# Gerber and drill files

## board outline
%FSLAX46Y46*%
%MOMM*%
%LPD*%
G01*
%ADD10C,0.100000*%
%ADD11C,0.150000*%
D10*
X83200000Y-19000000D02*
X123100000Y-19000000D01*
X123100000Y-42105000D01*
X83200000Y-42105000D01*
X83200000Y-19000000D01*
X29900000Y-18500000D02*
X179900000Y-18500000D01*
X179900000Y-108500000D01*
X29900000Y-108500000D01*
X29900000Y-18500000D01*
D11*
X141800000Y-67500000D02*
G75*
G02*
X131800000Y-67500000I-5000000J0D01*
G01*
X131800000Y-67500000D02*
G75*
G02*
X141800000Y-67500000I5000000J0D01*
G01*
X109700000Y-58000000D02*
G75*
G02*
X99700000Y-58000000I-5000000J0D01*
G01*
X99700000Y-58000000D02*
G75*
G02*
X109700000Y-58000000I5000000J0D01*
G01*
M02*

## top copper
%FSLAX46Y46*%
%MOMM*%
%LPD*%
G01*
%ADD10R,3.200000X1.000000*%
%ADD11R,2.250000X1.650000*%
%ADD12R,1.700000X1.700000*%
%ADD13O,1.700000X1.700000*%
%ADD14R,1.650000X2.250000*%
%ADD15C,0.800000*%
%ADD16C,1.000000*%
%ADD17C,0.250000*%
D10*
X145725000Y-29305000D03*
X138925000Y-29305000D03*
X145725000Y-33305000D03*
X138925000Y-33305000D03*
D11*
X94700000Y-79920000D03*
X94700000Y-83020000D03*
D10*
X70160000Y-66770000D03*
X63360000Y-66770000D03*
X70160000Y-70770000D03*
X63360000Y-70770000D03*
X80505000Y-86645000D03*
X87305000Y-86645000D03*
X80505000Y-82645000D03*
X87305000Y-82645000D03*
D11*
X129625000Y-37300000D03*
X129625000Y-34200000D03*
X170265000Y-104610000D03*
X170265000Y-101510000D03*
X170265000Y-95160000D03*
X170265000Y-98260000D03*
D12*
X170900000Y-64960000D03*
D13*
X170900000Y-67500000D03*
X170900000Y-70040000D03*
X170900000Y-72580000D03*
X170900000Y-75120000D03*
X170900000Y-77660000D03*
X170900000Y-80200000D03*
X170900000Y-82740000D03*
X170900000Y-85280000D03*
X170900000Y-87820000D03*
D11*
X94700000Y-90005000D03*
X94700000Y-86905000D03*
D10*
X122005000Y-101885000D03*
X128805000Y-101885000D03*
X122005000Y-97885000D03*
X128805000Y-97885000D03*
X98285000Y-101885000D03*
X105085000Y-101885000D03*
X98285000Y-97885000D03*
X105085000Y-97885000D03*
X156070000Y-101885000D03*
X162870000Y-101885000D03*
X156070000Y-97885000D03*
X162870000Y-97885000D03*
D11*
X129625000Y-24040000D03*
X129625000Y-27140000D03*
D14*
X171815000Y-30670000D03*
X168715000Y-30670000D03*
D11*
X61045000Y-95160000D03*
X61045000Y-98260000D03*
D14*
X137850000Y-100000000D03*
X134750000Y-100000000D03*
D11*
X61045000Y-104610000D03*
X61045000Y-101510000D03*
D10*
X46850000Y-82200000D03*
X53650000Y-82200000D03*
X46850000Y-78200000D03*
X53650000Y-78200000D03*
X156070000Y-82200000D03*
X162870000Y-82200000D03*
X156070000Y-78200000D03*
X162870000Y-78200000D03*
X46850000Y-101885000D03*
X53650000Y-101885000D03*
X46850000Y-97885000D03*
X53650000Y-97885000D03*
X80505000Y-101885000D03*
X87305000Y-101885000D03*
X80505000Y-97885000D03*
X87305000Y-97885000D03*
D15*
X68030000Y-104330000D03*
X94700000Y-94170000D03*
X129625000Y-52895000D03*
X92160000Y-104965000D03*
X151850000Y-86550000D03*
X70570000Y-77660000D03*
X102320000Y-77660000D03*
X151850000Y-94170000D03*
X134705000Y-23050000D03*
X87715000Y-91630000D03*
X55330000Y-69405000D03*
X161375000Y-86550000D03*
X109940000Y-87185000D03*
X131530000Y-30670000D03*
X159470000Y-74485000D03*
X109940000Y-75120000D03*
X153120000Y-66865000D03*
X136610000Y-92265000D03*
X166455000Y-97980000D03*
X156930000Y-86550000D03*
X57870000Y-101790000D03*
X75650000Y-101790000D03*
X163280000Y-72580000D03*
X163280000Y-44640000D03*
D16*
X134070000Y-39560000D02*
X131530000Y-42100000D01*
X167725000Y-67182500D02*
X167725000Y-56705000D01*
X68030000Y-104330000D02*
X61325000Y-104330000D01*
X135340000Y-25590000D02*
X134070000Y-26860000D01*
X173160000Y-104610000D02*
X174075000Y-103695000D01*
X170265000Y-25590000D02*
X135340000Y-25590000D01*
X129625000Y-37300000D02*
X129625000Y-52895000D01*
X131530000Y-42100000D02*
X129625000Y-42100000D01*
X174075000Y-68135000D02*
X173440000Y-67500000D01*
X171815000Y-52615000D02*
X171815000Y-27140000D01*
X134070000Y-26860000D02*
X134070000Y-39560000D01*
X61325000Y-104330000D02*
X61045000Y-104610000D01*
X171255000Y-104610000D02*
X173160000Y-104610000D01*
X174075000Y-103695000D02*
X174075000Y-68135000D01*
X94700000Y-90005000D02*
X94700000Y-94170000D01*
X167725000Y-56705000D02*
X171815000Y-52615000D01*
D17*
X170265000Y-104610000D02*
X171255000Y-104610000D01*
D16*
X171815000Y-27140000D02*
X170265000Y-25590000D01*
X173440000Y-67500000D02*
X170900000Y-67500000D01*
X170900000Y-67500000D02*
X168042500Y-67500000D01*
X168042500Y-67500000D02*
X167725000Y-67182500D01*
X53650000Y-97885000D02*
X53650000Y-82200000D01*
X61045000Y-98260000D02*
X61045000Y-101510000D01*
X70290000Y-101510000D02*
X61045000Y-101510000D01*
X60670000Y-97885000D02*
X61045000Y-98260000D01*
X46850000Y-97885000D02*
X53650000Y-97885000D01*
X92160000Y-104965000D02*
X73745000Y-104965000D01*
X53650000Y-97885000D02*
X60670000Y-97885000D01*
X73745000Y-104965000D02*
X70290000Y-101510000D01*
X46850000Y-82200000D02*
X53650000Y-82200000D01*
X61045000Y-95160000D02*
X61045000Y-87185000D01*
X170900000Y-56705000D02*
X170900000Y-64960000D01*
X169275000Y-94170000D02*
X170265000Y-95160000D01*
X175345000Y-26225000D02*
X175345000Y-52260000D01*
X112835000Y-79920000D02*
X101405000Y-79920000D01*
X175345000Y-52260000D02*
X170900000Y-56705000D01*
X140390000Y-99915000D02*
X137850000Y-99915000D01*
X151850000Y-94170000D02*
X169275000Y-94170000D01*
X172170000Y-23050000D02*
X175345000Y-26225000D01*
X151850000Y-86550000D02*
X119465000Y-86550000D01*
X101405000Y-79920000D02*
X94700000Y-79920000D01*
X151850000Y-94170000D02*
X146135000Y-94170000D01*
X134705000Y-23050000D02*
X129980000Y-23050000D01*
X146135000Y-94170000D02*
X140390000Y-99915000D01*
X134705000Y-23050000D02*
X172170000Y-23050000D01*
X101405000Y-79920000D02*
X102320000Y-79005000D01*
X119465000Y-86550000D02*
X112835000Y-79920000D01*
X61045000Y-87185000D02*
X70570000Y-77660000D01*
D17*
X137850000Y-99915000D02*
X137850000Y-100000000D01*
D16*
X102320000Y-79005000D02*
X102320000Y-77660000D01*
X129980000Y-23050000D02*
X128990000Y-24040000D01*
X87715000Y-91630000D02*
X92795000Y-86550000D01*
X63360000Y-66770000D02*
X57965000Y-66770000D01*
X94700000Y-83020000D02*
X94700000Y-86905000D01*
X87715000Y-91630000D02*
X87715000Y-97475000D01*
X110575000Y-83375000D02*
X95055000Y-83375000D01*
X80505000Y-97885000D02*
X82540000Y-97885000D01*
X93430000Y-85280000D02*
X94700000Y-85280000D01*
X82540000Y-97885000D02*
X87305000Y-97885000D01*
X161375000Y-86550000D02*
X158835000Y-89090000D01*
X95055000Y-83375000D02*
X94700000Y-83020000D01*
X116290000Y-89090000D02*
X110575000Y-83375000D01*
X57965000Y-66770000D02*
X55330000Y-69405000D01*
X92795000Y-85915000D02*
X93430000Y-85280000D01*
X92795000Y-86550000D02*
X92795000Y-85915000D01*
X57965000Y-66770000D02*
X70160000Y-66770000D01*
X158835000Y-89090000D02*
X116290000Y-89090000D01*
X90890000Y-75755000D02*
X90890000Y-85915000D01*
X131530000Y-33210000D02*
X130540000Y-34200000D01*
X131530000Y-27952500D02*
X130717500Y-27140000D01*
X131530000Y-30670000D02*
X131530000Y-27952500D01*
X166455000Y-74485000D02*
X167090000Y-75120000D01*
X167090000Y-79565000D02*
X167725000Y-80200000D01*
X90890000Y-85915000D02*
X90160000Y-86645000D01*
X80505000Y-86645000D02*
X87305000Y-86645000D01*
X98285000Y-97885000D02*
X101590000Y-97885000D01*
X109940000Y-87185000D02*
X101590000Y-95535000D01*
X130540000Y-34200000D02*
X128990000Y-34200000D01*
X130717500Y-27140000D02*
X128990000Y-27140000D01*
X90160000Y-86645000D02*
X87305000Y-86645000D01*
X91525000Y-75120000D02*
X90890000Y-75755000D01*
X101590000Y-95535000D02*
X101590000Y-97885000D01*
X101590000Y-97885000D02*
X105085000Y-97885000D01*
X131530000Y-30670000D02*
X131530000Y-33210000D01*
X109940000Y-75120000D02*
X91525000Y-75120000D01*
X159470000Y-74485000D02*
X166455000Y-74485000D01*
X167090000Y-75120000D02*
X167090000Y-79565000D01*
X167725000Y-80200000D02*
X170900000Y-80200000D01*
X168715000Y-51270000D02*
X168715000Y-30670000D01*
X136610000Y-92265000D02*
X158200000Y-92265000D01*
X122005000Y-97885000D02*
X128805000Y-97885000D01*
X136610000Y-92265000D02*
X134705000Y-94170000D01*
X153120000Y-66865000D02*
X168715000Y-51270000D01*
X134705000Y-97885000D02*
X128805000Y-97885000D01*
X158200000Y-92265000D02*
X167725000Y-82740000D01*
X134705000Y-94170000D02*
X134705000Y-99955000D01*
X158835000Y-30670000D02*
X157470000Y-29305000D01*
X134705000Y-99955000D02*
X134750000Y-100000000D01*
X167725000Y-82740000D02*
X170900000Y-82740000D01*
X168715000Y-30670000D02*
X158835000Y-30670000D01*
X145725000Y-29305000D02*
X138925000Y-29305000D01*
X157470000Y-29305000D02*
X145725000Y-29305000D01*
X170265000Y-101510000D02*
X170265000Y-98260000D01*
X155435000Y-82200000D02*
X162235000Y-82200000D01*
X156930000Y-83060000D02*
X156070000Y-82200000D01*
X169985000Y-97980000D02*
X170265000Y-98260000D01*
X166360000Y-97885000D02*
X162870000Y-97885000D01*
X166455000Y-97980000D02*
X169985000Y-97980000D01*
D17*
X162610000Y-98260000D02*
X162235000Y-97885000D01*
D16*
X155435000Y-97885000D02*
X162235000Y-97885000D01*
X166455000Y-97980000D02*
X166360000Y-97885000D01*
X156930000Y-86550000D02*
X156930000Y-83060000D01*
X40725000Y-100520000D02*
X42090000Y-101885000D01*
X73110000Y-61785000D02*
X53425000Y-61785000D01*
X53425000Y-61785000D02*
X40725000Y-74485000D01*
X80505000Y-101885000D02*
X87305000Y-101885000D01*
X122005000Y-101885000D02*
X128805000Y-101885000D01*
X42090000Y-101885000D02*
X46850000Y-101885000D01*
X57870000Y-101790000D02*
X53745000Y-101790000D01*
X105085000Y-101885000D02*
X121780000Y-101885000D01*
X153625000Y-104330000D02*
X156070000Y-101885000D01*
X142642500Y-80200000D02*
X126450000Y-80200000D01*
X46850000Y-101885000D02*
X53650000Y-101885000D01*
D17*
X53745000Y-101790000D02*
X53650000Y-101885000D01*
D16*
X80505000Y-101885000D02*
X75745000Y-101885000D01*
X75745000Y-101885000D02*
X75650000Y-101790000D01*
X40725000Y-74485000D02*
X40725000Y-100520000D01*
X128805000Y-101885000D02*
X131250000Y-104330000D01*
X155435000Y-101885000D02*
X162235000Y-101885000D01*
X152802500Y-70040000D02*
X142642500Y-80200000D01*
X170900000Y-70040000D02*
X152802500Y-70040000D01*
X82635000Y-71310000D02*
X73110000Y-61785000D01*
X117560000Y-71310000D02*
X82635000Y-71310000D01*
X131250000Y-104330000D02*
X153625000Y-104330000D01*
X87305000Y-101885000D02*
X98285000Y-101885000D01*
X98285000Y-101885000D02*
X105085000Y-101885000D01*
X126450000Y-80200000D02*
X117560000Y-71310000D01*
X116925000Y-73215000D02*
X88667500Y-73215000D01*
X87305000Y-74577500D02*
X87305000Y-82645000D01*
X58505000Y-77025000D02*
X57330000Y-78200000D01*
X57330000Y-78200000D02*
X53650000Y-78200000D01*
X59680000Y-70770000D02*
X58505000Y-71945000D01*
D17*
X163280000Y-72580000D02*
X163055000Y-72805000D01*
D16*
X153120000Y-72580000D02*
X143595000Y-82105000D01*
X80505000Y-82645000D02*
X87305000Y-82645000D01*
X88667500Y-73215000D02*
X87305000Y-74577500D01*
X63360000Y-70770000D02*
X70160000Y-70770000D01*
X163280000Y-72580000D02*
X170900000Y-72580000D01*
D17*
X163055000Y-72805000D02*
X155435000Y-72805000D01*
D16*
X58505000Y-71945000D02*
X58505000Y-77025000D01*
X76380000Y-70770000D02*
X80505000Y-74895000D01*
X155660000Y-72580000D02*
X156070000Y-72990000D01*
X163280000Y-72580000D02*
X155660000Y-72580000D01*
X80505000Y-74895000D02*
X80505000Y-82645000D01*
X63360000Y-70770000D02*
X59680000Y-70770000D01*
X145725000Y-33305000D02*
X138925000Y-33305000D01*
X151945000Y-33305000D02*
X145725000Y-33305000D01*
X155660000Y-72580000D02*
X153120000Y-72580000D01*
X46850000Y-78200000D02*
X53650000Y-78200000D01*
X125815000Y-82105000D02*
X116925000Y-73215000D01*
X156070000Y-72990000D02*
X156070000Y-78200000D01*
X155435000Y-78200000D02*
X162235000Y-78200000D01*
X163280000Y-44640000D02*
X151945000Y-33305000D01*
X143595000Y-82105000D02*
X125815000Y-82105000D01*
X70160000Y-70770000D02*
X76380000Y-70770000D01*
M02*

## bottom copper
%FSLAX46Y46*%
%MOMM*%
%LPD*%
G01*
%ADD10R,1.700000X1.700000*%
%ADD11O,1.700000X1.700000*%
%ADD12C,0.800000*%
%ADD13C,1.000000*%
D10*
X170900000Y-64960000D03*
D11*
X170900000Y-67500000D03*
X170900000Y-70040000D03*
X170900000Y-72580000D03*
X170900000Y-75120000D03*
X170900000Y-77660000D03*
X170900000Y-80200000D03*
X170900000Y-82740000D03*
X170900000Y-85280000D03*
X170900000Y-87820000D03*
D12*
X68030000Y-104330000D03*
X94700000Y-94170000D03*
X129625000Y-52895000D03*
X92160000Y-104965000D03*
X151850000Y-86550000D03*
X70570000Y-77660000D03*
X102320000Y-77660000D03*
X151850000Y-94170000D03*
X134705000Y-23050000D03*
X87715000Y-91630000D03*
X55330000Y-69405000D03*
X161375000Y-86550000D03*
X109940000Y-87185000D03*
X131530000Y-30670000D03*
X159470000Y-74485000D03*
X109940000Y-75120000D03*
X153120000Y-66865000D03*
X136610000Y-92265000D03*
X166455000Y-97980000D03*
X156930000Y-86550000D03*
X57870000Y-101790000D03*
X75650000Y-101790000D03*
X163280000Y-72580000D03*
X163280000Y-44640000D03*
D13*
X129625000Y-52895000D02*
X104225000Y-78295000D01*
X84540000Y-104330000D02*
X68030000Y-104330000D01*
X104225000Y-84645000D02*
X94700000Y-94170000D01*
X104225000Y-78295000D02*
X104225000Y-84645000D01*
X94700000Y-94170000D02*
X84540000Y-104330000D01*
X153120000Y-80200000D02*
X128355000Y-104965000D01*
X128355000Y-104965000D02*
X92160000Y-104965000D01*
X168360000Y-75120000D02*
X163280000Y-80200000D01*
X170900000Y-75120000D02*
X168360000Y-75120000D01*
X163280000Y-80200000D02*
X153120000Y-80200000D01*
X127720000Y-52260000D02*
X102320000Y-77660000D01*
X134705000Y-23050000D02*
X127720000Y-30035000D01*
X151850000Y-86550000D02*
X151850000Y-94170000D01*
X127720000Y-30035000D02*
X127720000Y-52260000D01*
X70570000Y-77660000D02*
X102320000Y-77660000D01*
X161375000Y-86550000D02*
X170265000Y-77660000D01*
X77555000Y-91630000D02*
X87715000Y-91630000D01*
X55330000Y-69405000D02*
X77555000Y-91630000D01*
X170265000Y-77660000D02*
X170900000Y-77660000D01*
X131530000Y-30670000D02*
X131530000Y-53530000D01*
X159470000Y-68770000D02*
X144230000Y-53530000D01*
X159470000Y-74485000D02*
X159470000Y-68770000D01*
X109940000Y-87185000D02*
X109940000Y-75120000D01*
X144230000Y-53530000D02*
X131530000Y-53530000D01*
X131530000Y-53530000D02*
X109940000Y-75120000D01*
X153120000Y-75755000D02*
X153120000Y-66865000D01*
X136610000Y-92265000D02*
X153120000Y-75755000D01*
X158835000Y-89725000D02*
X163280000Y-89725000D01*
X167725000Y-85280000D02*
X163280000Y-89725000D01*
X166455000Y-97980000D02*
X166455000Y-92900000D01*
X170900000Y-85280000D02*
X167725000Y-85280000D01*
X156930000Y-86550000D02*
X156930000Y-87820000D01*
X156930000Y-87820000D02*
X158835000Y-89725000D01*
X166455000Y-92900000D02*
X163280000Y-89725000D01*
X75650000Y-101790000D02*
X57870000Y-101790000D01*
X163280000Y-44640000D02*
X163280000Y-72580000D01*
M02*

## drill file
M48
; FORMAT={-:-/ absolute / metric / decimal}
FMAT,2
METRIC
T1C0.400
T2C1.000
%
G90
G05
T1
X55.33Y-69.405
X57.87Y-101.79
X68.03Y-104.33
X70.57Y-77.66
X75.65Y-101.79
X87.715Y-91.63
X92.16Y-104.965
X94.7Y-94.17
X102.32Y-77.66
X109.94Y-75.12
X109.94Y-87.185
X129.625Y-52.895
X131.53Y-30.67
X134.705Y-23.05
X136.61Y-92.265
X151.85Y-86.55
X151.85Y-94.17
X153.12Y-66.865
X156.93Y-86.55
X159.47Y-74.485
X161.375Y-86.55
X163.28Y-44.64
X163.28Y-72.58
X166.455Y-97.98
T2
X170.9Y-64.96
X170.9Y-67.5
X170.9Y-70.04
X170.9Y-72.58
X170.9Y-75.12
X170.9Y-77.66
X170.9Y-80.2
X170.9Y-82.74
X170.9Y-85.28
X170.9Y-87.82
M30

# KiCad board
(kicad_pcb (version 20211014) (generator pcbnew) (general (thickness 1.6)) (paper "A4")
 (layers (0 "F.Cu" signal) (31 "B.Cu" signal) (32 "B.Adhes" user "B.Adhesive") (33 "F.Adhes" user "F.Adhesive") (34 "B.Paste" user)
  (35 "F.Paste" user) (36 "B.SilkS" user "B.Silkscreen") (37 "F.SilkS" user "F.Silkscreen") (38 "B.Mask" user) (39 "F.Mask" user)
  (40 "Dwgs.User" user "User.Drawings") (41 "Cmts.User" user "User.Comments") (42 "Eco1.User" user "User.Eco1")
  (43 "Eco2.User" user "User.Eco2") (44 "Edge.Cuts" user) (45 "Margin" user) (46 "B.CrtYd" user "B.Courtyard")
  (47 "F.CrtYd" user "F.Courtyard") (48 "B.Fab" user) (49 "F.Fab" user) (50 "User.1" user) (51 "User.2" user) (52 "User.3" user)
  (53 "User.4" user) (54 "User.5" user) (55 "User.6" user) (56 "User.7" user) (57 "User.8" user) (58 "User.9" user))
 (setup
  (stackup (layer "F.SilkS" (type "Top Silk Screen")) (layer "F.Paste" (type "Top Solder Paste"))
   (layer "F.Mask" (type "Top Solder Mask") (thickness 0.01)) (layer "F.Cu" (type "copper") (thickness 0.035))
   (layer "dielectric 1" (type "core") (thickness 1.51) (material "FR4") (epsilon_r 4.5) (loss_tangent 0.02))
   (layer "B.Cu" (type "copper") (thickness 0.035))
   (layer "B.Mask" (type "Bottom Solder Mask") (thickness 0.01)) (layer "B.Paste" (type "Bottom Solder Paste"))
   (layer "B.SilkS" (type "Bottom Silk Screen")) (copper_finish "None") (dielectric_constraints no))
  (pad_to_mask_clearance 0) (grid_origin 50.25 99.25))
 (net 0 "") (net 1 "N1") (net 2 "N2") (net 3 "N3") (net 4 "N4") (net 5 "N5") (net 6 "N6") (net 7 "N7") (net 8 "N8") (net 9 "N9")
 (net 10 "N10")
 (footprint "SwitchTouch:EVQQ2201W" (layer "F.Cu") (at 142.325 31.305 180)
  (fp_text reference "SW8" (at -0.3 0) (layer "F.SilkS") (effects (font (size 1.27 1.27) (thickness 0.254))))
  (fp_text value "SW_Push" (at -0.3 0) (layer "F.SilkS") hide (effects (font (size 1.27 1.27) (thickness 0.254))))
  (pad "A1" smd rect locked (at -3.4 2 270) (size 1 3.2) (layers "F.Cu" "F.Paste" "F.Mask") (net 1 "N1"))
  (pad "A2" smd rect locked (at 3.4 2 270) (size 1 3.2) (layers "F.Cu" "F.Paste" "F.Mask") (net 1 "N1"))
  (pad "B1" smd rect locked (at -3.4 -2 270) (size 1 3.2) (layers "F.Cu" "F.Paste" "F.Mask") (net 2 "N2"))
  (pad "B2" smd rect locked (at 3.4 -2 270) (size 1 3.2) (layers "F.Cu" "F.Paste" "F.Mask") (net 2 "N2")))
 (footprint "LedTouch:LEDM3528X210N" (layer "F.Cu") (at 94.7 81.47 -90)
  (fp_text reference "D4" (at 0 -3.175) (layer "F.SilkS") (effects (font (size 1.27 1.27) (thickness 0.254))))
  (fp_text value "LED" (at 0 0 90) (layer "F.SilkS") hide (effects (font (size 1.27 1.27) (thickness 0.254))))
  (pad "1" smd rect locked (at -1.55 0 270) (size 1.65 2.25) (layers "F.Cu" "F.Paste" "F.Mask") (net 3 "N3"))
  (pad "2" smd rect locked (at 1.55 0 270) (size 1.65 2.25) (layers "F.Cu" "F.Paste" "F.Mask") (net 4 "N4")))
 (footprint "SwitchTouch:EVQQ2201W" (layer "F.Cu") (at 66.76 68.77 180)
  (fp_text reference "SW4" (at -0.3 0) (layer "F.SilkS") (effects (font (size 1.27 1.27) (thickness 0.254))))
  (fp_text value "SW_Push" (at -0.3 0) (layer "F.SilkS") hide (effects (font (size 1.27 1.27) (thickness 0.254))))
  (pad "A1" smd rect locked (at -3.4 2 270) (size 1 3.2) (layers "F.Cu" "F.Paste" "F.Mask") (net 4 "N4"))
  (pad "A2" smd rect locked (at 3.4 2 270) (size 1 3.2) (layers "F.Cu" "F.Paste" "F.Mask") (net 4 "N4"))
  (pad "B1" smd rect locked (at -3.4 -2 270) (size 1 3.2) (layers "F.Cu" "F.Paste" "F.Mask") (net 2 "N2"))
  (pad "B2" smd rect locked (at 3.4 -2 270) (size 1 3.2) (layers "F.Cu" "F.Paste" "F.Mask") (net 2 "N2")))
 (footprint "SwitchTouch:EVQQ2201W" (layer "F.Cu") (at 83.905 84.645)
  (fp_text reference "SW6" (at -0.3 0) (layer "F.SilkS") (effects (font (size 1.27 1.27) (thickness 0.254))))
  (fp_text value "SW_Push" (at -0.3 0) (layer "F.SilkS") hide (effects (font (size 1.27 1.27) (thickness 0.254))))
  (pad "A1" smd rect locked (at -3.4 2 90) (size 1 3.2) (layers "F.Cu" "F.Paste" "F.Mask") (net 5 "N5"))
  (pad "A2" smd rect locked (at 3.4 2 90) (size 1 3.2) (layers "F.Cu" "F.Paste" "F.Mask") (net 5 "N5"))
  (pad "B1" smd rect locked (at -3.4 -2 90) (size 1 3.2) (layers "F.Cu" "F.Paste" "F.Mask") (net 2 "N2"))
  (pad "B2" smd rect locked (at 3.4 -2 90) (size 1 3.2) (layers "F.Cu" "F.Paste" "F.Mask") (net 2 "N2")))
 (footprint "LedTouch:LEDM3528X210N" (layer "F.Cu") (at 129.625 35.75 90)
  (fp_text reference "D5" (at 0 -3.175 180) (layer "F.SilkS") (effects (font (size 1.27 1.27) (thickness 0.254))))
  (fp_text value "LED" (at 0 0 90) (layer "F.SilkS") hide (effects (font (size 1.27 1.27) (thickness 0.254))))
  (pad "1" smd rect locked (at -1.55 0 90) (size 1.65 2.25) (layers "F.Cu" "F.Paste" "F.Mask") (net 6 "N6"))
  (pad "2" smd rect locked (at 1.55 0 90) (size 1.65 2.25) (layers "F.Cu" "F.Paste" "F.Mask") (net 5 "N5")))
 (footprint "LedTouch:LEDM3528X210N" (layer "F.Cu") (at 170.265 103.06 90)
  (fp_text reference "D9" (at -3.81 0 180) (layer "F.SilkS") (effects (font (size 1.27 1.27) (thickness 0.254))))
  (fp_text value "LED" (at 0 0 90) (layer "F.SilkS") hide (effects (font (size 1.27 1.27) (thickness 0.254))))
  (pad "1" smd rect locked (at -1.55 0 90) (size 1.65 2.25) (layers "F.Cu" "F.Paste" "F.Mask") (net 6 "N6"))
  (pad "2" smd rect locked (at 1.55 0 90) (size 1.65 2.25) (layers "F.Cu" "F.Paste" "F.Mask") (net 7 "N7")))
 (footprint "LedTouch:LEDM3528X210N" (layer "F.Cu") (at 170.265 96.71 -90)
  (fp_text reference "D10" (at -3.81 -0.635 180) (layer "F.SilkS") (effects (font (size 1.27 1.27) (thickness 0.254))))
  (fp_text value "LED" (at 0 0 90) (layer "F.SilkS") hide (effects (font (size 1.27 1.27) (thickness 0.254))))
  (pad "1" smd rect locked (at -1.55 0 270) (size 1.65 2.25) (layers "F.Cu" "F.Paste" "F.Mask") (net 3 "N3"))
  (pad "2" smd rect locked (at 1.55 0 270) (size 1.65 2.25) (layers "F.Cu" "F.Paste" "F.Mask") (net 7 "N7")))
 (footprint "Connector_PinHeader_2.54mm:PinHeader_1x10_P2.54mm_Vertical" (layer "F.Cu") (at 170.9 64.96)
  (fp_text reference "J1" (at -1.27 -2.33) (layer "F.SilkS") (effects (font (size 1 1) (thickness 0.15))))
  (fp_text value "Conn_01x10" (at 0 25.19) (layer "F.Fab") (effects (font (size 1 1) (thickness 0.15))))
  (pad "1" thru_hole rect (at 0 0) (size 1.7 1.7) (drill 1) (layers *.Cu *.Mask) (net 3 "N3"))
  (pad "2" thru_hole oval (at 0 2.54) (size 1.7 1.7) (drill 1) (layers *.Cu *.Mask) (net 6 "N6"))
  (pad "3" thru_hole oval (at 0 5.08) (size 1.7 1.7) (drill 1) (layers *.Cu *.Mask) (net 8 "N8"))
  (pad "4" thru_hole oval (at 0 7.62) (size 1.7 1.7) (drill 1) (layers *.Cu *.Mask) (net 2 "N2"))
  (pad "5" thru_hole oval (at 0 10.16) (size 1.7 1.7) (drill 1) (layers *.Cu *.Mask) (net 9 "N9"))
  (pad "6" thru_hole oval (at 0 12.7) (size 1.7 1.7) (drill 1) (layers *.Cu *.Mask) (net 4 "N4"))
  (pad "7" thru_hole oval (at 0 15.24) (size 1.7 1.7) (drill 1) (layers *.Cu *.Mask) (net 5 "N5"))
  (pad "8" thru_hole oval (at 0 17.78) (size 1.7 1.7) (drill 1) (layers *.Cu *.Mask) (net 1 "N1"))
  (pad "9" thru_hole oval (at 0 20.32) (size 1.7 1.7) (drill 1) (layers *.Cu *.Mask) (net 7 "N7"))
  (pad "10" thru_hole oval (at 0 22.86) (size 1.7 1.7) (drill 1) (layers *.Cu *.Mask) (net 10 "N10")))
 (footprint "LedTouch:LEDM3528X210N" (layer "F.Cu") (at 94.7 88.455 90)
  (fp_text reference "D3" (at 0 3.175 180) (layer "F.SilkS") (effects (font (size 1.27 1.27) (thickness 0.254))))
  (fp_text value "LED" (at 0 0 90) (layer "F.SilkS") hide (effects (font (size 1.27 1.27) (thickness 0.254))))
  (pad "1" smd rect locked (at -1.55 0 90) (size 1.65 2.25) (layers "F.Cu" "F.Paste" "F.Mask") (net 6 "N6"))
  (pad "2" smd rect locked (at 1.55 0 90) (size 1.65 2.25) (layers "F.Cu" "F.Paste" "F.Mask") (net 4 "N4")))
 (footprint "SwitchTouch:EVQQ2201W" (layer "F.Cu") (at 125.405 99.885)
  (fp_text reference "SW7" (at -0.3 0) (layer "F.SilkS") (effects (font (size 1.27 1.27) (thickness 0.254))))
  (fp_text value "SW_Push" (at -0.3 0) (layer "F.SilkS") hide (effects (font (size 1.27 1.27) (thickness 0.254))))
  (pad "A1" smd rect locked (at -3.4 2 90) (size 1 3.2) (layers "F.Cu" "F.Paste" "F.Mask") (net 8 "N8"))
  (pad "A2" smd rect locked (at 3.4 2 90) (size 1 3.2) (layers "F.Cu" "F.Paste" "F.Mask") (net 8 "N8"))
  (pad "B1" smd rect locked (at -3.4 -2 90) (size 1 3.2) (layers "F.Cu" "F.Paste" "F.Mask") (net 1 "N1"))
  (pad "B2" smd rect locked (at 3.4 -2 90) (size 1 3.2) (layers "F.Cu" "F.Paste" "F.Mask") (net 1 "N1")))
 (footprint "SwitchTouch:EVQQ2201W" (layer "F.Cu") (at 101.685 99.885)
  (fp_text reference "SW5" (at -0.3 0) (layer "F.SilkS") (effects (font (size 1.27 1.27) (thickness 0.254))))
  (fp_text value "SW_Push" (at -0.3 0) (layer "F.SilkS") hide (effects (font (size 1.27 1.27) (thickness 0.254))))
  (pad "A1" smd rect locked (at -3.4 2 90) (size 1 3.2) (layers "F.Cu" "F.Paste" "F.Mask") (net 8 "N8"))
  (pad "A2" smd rect locked (at 3.4 2 90) (size 1 3.2) (layers "F.Cu" "F.Paste" "F.Mask") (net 8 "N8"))
  (pad "B1" smd rect locked (at -3.4 -2 90) (size 1 3.2) (layers "F.Cu" "F.Paste" "F.Mask") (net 5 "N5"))
  (pad "B2" smd rect locked (at 3.4 -2 90) (size 1 3.2) (layers "F.Cu" "F.Paste" "F.Mask") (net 5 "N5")))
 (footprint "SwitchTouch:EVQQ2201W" (layer "F.Cu") (at 159.47 99.885)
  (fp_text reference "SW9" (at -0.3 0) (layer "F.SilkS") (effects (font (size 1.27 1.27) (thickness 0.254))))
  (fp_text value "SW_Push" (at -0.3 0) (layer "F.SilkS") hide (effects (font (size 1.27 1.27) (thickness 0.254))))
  (pad "A1" smd rect locked (at -3.4 2 90) (size 1 3.2) (layers "F.Cu" "F.Paste" "F.Mask") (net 8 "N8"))
  (pad "A2" smd rect locked (at 3.4 2 90) (size 1 3.2) (layers "F.Cu" "F.Paste" "F.Mask") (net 8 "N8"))
  (pad "B1" smd rect locked (at -3.4 -2 90) (size 1 3.2) (layers "F.Cu" "F.Paste" "F.Mask") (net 7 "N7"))
  (pad "B2" smd rect locked (at 3.4 -2 90) (size 1 3.2) (layers "F.Cu" "F.Paste" "F.Mask") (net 7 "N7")))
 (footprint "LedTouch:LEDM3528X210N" (layer "F.Cu") (at 129.625 25.59 -90)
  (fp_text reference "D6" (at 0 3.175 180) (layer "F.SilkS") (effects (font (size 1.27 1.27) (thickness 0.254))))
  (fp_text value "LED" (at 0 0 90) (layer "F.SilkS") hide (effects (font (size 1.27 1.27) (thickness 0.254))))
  (pad "1" smd rect locked (at -1.55 0 270) (size 1.65 2.25) (layers "F.Cu" "F.Paste" "F.Mask") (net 3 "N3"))
  (pad "2" smd rect locked (at 1.55 0 270) (size 1.65 2.25) (layers "F.Cu" "F.Paste" "F.Mask") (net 5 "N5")))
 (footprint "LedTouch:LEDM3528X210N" (layer "F.Cu") (at 170.265 30.67 180)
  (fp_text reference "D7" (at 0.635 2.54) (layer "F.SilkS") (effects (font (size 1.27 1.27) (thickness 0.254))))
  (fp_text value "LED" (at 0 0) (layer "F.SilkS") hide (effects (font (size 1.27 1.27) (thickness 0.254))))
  (pad "1" smd rect locked (at -1.55 0 180) (size 1.65 2.25) (layers "F.Cu" "F.Paste" "F.Mask") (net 6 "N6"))
  (pad "2" smd rect locked (at 1.55 0 180) (size 1.65 2.25) (layers "F.Cu" "F.Paste" "F.Mask") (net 1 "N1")))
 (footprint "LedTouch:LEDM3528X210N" (layer "F.Cu") (at 61.045 96.71 -90)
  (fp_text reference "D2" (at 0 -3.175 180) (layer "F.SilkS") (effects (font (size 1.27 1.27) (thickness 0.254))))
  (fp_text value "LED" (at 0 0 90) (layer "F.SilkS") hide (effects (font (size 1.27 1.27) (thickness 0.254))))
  (pad "1" smd rect locked (at -1.55 0 270) (size 1.65 2.25) (layers "F.Cu" "F.Paste" "F.Mask") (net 3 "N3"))
  (pad "2" smd rect locked (at 1.55 0 270) (size 1.65 2.25) (layers "F.Cu" "F.Paste" "F.Mask") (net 9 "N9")))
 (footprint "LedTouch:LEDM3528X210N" (layer "F.Cu") (at 136.3 100 180)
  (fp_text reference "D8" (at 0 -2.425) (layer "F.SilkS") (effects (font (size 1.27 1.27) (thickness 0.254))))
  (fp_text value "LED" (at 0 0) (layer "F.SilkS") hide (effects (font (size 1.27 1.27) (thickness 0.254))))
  (pad "1" smd rect locked (at -1.55 0 180) (size 1.65 2.25) (layers "F.Cu" "F.Paste" "F.Mask") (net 3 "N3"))
  (pad "2" smd rect locked (at 1.55 0 180) (size 1.65 2.25) (layers "F.Cu" "F.Paste" "F.Mask") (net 1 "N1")))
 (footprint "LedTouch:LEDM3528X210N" (layer "F.Cu") (at 61.045 103.06 90)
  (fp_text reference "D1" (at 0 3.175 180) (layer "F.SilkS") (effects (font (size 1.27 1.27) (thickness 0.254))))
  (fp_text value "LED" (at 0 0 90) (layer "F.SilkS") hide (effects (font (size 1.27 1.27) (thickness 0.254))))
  (pad "1" smd rect locked (at -1.55 0 90) (size 1.65 2.25) (layers "F.Cu" "F.Paste" "F.Mask") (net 6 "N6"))
  (pad "2" smd rect locked (at 1.55 0 90) (size 1.65 2.25) (layers "F.Cu" "F.Paste" "F.Mask") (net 9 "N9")))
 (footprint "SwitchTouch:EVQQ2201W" (layer "F.Cu") (at 50.25 80.2)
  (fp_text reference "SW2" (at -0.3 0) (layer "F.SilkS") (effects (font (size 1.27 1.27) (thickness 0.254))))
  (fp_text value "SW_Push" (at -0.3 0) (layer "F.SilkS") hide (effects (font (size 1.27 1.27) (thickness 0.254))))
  (pad "A1" smd rect locked (at -3.4 2 90) (size 1 3.2) (layers "F.Cu" "F.Paste" "F.Mask") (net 9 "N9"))
  (pad "A2" smd rect locked (at 3.4 2 90) (size 1 3.2) (layers "F.Cu" "F.Paste" "F.Mask") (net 9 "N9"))
  (pad "B1" smd rect locked (at -3.4 -2 90) (size 1 3.2) (layers "F.Cu" "F.Paste" "F.Mask") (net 2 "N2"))
  (pad "B2" smd rect locked (at 3.4 -2 90) (size 1 3.2) (layers "F.Cu" "F.Paste" "F.Mask") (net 2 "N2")))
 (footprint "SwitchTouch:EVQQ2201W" (layer "F.Cu") (at 159.47 80.2)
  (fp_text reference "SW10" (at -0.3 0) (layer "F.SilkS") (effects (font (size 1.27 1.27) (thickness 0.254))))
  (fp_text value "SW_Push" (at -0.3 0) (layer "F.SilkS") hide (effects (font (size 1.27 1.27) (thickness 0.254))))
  (pad "A1" smd rect locked (at -3.4 2 90) (size 1 3.2) (layers "F.Cu" "F.Paste" "F.Mask") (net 7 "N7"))
  (pad "A2" smd rect locked (at 3.4 2 90) (size 1 3.2) (layers "F.Cu" "F.Paste" "F.Mask") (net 7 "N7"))
  (pad "B1" smd rect locked (at -3.4 -2 90) (size 1 3.2) (layers "F.Cu" "F.Paste" "F.Mask") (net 2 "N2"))
  (pad "B2" smd rect locked (at 3.4 -2 90) (size 1 3.2) (layers "F.Cu" "F.Paste" "F.Mask") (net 2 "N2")))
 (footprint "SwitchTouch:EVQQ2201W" (layer "F.Cu") (at 50.25 99.885)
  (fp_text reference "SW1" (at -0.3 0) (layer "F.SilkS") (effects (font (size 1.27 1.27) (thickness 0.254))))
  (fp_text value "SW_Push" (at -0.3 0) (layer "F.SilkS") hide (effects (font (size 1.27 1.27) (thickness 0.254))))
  (pad "A1" smd rect locked (at -3.4 2 90) (size 1 3.2) (layers "F.Cu" "F.Paste" "F.Mask") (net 8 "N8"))
  (pad "A2" smd rect locked (at 3.4 2 90) (size 1 3.2) (layers "F.Cu" "F.Paste" "F.Mask") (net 8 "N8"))
  (pad "B1" smd rect locked (at -3.4 -2 90) (size 1 3.2) (layers "F.Cu" "F.Paste" "F.Mask") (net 9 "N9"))
  (pad "B2" smd rect locked (at 3.4 -2 90) (size 1 3.2) (layers "F.Cu" "F.Paste" "F.Mask") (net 9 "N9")))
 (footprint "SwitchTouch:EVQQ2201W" (layer "F.Cu") (at 83.905 99.885)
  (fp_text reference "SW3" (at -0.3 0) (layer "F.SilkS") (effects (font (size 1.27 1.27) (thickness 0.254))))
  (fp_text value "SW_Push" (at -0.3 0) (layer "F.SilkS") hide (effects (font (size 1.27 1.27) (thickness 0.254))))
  (pad "A1" smd rect locked (at -3.4 2 90) (size 1 3.2) (layers "F.Cu" "F.Paste" "F.Mask") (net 8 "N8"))
  (pad "A2" smd rect locked (at 3.4 2 90) (size 1 3.2) (layers "F.Cu" "F.Paste" "F.Mask") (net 8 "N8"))
  (pad "B1" smd rect locked (at -3.4 -2 90) (size 1 3.2) (layers "F.Cu" "F.Paste" "F.Mask") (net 4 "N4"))
  (pad "B2" smd rect locked (at 3.4 -2 90) (size 1 3.2) (layers "F.Cu" "F.Paste" "F.Mask") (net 4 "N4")))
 (gr_rect (start 83.2 19) (end 123.1 42.105) (layer "Edge.Cuts") (width 0.1) (fill none))
 (gr_rect (start 29.9 18.5) (end 179.9 108.5) (layer "Edge.Cuts") (width 0.1) (fill none))
 (gr_circle (center 136.8 67.5) (end 141.8 67.5) (layer "Edge.Cuts") (width 0.15) (fill none))
 (gr_circle (center 104.7 58) (end 109.7 58) (layer "Edge.Cuts") (width 0.15) (fill none))
 (segment (start 134.07 39.56) (end 131.53 42.1) (width 1) (layer "F.Cu") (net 6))
 (segment (start 167.725 67.1825) (end 167.725 56.705) (width 1) (layer "F.Cu") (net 6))
 (segment (start 68.03 104.33) (end 61.325 104.33) (width 1) (layer "F.Cu") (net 6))
 (segment (start 135.34 25.59) (end 134.07 26.86) (width 1) (layer "F.Cu") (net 6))
 (segment (start 173.16 104.61) (end 174.075 103.695) (width 1) (layer "F.Cu") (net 6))
 (segment (start 170.265 25.59) (end 135.34 25.59) (width 1) (layer "F.Cu") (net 6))
 (segment (start 129.625 37.3) (end 129.625 52.895) (width 1) (layer "F.Cu") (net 6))
 (segment (start 131.53 42.1) (end 129.625 42.1) (width 1) (layer "F.Cu") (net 6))
 (segment (start 174.075 68.135) (end 173.44 67.5) (width 1) (layer "F.Cu") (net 6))
 (segment (start 171.815 52.615) (end 171.815 27.14) (width 1) (layer "F.Cu") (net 6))
 (segment (start 134.07 26.86) (end 134.07 39.56) (width 1) (layer "F.Cu") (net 6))
 (segment (start 61.325 104.33) (end 61.045 104.61) (width 1) (layer "F.Cu") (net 6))
 (segment (start 171.255 104.61) (end 173.16 104.61) (width 1) (layer "F.Cu") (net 6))
 (segment (start 174.075 103.695) (end 174.075 68.135) (width 1) (layer "F.Cu") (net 6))
 (segment (start 94.7 90.005) (end 94.7 94.17) (width 1) (layer "F.Cu") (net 6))
 (segment (start 167.725 56.705) (end 171.815 52.615) (width 1) (layer "F.Cu") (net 6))
 (segment (start 170.265 104.61) (end 171.255 104.61) (width 0.25) (layer "F.Cu") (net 6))
 (segment (start 171.815 27.14) (end 170.265 25.59) (width 1) (layer "F.Cu") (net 6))
 (segment (start 173.44 67.5) (end 170.9 67.5) (width 1) (layer "F.Cu") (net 6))
 (segment (start 170.9 67.5) (end 168.0425 67.5) (width 1) (layer "F.Cu") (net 6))
 (segment (start 168.0425 67.5) (end 167.725 67.1825) (width 1) (layer "F.Cu") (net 6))
 (via (at 68.03 104.33) (size 0.8) (drill 0.4) (layers "F.Cu" "B.Cu") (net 6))
 (via (at 94.7 94.17) (size 0.8) (drill 0.4) (layers "F.Cu" "B.Cu") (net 6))
 (via (at 129.625 52.895) (size 0.8) (drill 0.4) (layers "F.Cu" "B.Cu") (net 6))
 (segment (start 129.625 52.895) (end 104.225 78.295) (width 1) (layer "B.Cu") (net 6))
 (segment (start 84.54 104.33) (end 68.03 104.33) (width 1) (layer "B.Cu") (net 6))
 (segment (start 104.225 84.645) (end 94.7 94.17) (width 1) (layer "B.Cu") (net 6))
 (segment (start 104.225 78.295) (end 104.225 84.645) (width 1) (layer "B.Cu") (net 6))
 (segment (start 94.7 94.17) (end 84.54 104.33) (width 1) (layer "B.Cu") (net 6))
 (segment (start 53.65 97.885) (end 53.65 82.2) (width 1) (layer "F.Cu") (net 9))
 (segment (start 61.045 98.26) (end 61.045 101.51) (width 1) (layer "F.Cu") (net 9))
 (segment (start 70.29 101.51) (end 61.045 101.51) (width 1) (layer "F.Cu") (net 9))
 (segment (start 60.67 97.885) (end 61.045 98.26) (width 1) (layer "F.Cu") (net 9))
 (segment (start 46.85 97.885) (end 53.65 97.885) (width 1) (layer "F.Cu") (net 9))
 (segment (start 92.16 104.965) (end 73.745 104.965) (width 1) (layer "F.Cu") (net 9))
 (segment (start 53.65 97.885) (end 60.67 97.885) (width 1) (layer "F.Cu") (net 9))
 (segment (start 73.745 104.965) (end 70.29 101.51) (width 1) (layer "F.Cu") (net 9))
 (segment (start 46.85 82.2) (end 53.65 82.2) (width 1) (layer "F.Cu") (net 9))
 (via (at 92.16 104.965) (size 0.8) (drill 0.4) (layers "F.Cu" "B.Cu") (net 9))
 (segment (start 153.12 80.2) (end 128.355 104.965) (width 1) (layer "B.Cu") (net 9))
 (segment (start 128.355 104.965) (end 92.16 104.965) (width 1) (layer "B.Cu") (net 9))
 (segment (start 168.36 75.12) (end 163.28 80.2) (width 1) (layer "B.Cu") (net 9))
 (segment (start 170.9 75.12) (end 168.36 75.12) (width 1) (layer "B.Cu") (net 9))
 (segment (start 163.28 80.2) (end 153.12 80.2) (width 1) (layer "B.Cu") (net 9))
 (segment (start 61.045 95.16) (end 61.045 87.185) (width 1) (layer "F.Cu") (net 3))
 (segment (start 170.9 56.705) (end 170.9 64.96) (width 1) (layer "F.Cu") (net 3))
 (segment (start 169.275 94.17) (end 170.265 95.16) (width 1) (layer "F.Cu") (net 3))
 (segment (start 175.345 26.225) (end 175.345 52.26) (width 1) (layer "F.Cu") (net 3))
 (segment (start 112.835 79.92) (end 101.405 79.92) (width 1) (layer "F.Cu") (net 3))
 (segment (start 175.345 52.26) (end 170.9 56.705) (width 1) (layer "F.Cu") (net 3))
 (segment (start 140.39 99.915) (end 137.85 99.915) (width 1) (layer "F.Cu") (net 3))
 (segment (start 151.85 94.17) (end 169.275 94.17) (width 1) (layer "F.Cu") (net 3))
 (segment (start 172.17 23.05) (end 175.345 26.225) (width 1) (layer "F.Cu") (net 3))
 (segment (start 151.85 86.55) (end 119.465 86.55) (width 1) (layer "F.Cu") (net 3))
 (segment (start 101.405 79.92) (end 94.7 79.92) (width 1) (layer "F.Cu") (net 3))
 (segment (start 151.85 94.17) (end 146.135 94.17) (width 1) (layer "F.Cu") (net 3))
 (segment (start 134.705 23.05) (end 129.98 23.05) (width 1) (layer "F.Cu") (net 3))
 (segment (start 146.135 94.17) (end 140.39 99.915) (width 1) (layer "F.Cu") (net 3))
 (segment (start 134.705 23.05) (end 172.17 23.05) (width 1) (layer "F.Cu") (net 3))
 (segment (start 101.405 79.92) (end 102.32 79.005) (width 1) (layer "F.Cu") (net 3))
 (segment (start 119.465 86.55) (end 112.835 79.92) (width 1) (layer "F.Cu") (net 3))
 (segment (start 61.045 87.185) (end 70.57 77.66) (width 1) (layer "F.Cu") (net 3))
 (segment (start 137.85 99.915) (end 137.85 100) (width 0.25) (layer "F.Cu") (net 3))
 (segment (start 102.32 79.005) (end 102.32 77.66) (width 1) (layer "F.Cu") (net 3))
 (segment (start 129.98 23.05) (end 128.99 24.04) (width 1) (layer "F.Cu") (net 3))
 (via (at 151.85 86.55) (size 0.8) (drill 0.4) (layers "F.Cu" "B.Cu") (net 3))
 (via (at 70.57 77.66) (size 0.8) (drill 0.4) (layers "F.Cu" "B.Cu") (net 3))
 (via (at 102.32 77.66) (size 0.8) (drill 0.4) (layers "F.Cu" "B.Cu") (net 3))
 (via (at 151.85 94.17) (size 0.8) (drill 0.4) (layers "F.Cu" "B.Cu") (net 3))
 (via (at 134.705 23.05) (size 0.8) (drill 0.4) (layers "F.Cu" "B.Cu") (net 3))
 (segment (start 127.72 52.26) (end 102.32 77.66) (width 1) (layer "B.Cu") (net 3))
 (segment (start 134.705 23.05) (end 127.72 30.035) (width 1) (layer "B.Cu") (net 3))
 (segment (start 151.85 86.55) (end 151.85 94.17) (width 1) (layer "B.Cu") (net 3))
 (segment (start 127.72 30.035) (end 127.72 52.26) (width 1) (layer "B.Cu") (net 3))
 (segment (start 70.57 77.66) (end 102.32 77.66) (width 1) (layer "B.Cu") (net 3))
 (segment (start 87.715 91.63) (end 92.795 86.55) (width 1) (layer "F.Cu") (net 4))
 (segment (start 63.36 66.77) (end 57.965 66.77) (width 1) (layer "F.Cu") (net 4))
 (segment (start 94.7 83.02) (end 94.7 86.905) (width 1) (layer "F.Cu") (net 4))
 (segment (start 87.715 91.63) (end 87.715 97.475) (width 1) (layer "F.Cu") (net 4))
 (segment (start 110.575 83.375) (end 95.055 83.375) (width 1) (layer "F.Cu") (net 4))
 (segment (start 80.505 97.885) (end 82.54 97.885) (width 1) (layer "F.Cu") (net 4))
 (segment (start 93.43 85.28) (end 94.7 85.28) (width 1) (layer "F.Cu") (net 4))
 (segment (start 82.54 97.885) (end 87.305 97.885) (width 1) (layer "F.Cu") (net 4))
 (segment (start 161.375 86.55) (end 158.835 89.09) (width 1) (layer "F.Cu") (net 4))
 (segment (start 95.055 83.375) (end 94.7 83.02) (width 1) (layer "F.Cu") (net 4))
 (segment (start 116.29 89.09) (end 110.575 83.375) (width 1) (layer "F.Cu") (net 4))
 (segment (start 57.965 66.77) (end 55.33 69.405) (width 1) (layer "F.Cu") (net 4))
 (segment (start 92.795 85.915) (end 93.43 85.28) (width 1) (layer "F.Cu") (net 4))
 (segment (start 92.795 86.55) (end 92.795 85.915) (width 1) (layer "F.Cu") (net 4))
 (segment (start 57.965 66.77) (end 70.16 66.77) (width 1) (layer "F.Cu") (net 4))
 (segment (start 158.835 89.09) (end 116.29 89.09) (width 1) (layer "F.Cu") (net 4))
 (via (at 87.715 91.63) (size 0.8) (drill 0.4) (layers "F.Cu" "B.Cu") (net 4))
 (via (at 55.33 69.405) (size 0.8) (drill 0.4) (layers "F.Cu" "B.Cu") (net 4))
 (via (at 161.375 86.55) (size 0.8) (drill 0.4) (layers "F.Cu" "B.Cu") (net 4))
 (segment (start 161.375 86.55) (end 170.265 77.66) (width 1) (layer "B.Cu") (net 4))
 (segment (start 77.555 91.63) (end 87.715 91.63) (width 1) (layer "B.Cu") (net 4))
 (segment (start 55.33 69.405) (end 77.555 91.63) (width 1) (layer "B.Cu") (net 4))
 (segment (start 170.265 77.66) (end 170.9 77.66) (width 1) (layer "B.Cu") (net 4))
 (segment (start 90.89 75.755) (end 90.89 85.915) (width 1) (layer "F.Cu") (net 5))
 (segment (start 131.53 33.21) (end 130.54 34.2) (width 1) (layer "F.Cu") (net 5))
 (segment (start 131.53 27.9525) (end 130.7175 27.14) (width 1) (layer "F.Cu") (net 5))
 (segment (start 131.53 30.67) (end 131.53 27.9525) (width 1) (layer "F.Cu") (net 5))
 (segment (start 166.455 74.485) (end 167.09 75.12) (width 1) (layer "F.Cu") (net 5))
 (segment (start 167.09 79.565) (end 167.725 80.2) (width 1) (layer "F.Cu") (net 5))
 (segment (start 90.89 85.915) (end 90.16 86.645) (width 1) (layer "F.Cu") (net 5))
 (segment (start 80.505 86.645) (end 87.305 86.645) (width 1) (layer "F.Cu") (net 5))
 (segment (start 98.285 97.885) (end 101.59 97.885) (width 1) (layer "F.Cu") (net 5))
 (segment (start 109.94 87.185) (end 101.59 95.535) (width 1) (layer "F.Cu") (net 5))
 (segment (start 130.54 34.2) (end 128.99 34.2) (width 1) (layer "F.Cu") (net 5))
 (segment (start 130.7175 27.14) (end 128.99 27.14) (width 1) (layer "F.Cu") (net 5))
 (segment (start 90.16 86.645) (end 87.305 86.645) (width 1) (layer "F.Cu") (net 5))
 (segment (start 91.525 75.12) (end 90.89 75.755) (width 1) (layer "F.Cu") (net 5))
 (segment (start 101.59 95.535) (end 101.59 97.885) (width 1) (layer "F.Cu") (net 5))
 (segment (start 101.59 97.885) (end 105.085 97.885) (width 1) (layer "F.Cu") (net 5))
 (segment (start 131.53 30.67) (end 131.53 33.21) (width 1) (layer "F.Cu") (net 5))
 (segment (start 109.94 75.12) (end 91.525 75.12) (width 1) (layer "F.Cu") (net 5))
 (segment (start 159.47 74.485) (end 166.455 74.485) (width 1) (layer "F.Cu") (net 5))
 (segment (start 167.09 75.12) (end 167.09 79.565) (width 1) (layer "F.Cu") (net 5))
 (segment (start 167.725 80.2) (end 170.9 80.2) (width 1) (layer "F.Cu") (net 5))
 (via (at 109.94 87.185) (size 0.8) (drill 0.4) (layers "F.Cu" "B.Cu") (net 5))
 (via (at 131.53 30.67) (size 0.8) (drill 0.4) (layers "F.Cu" "B.Cu") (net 5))
 (via (at 159.47 74.485) (size 0.8) (drill 0.4) (layers "F.Cu" "B.Cu") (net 5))
 (via (at 109.94 75.12) (size 0.8) (drill 0.4) (layers "F.Cu" "B.Cu") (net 5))
 (segment (start 131.53 30.67) (end 131.53 53.53) (width 1) (layer "B.Cu") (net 5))
 (segment (start 159.47 68.77) (end 144.23 53.53) (width 1) (layer "B.Cu") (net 5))
 (segment (start 159.47 74.485) (end 159.47 68.77) (width 1) (layer "B.Cu") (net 5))
 (segment (start 109.94 87.185) (end 109.94 75.12) (width 1) (layer "B.Cu") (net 5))
 (segment (start 144.23 53.53) (end 131.53 53.53) (width 1) (layer "B.Cu") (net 5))
 (segment (start 131.53 53.53) (end 109.94 75.12) (width 1) (layer "B.Cu") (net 5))
 (segment (start 168.715 51.27) (end 168.715 30.67) (width 1) (layer "F.Cu") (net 1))
 (segment (start 136.61 92.265) (end 158.2 92.265) (width 1) (layer "F.Cu") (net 1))
 (segment (start 122.005 97.885) (end 128.805 97.885) (width 1) (layer "F.Cu") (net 1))
 (segment (start 136.61 92.265) (end 134.705 94.17) (width 1) (layer "F.Cu") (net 1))
 (segment (start 153.12 66.865) (end 168.715 51.27) (width 1) (layer "F.Cu") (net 1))
 (segment (start 134.705 97.885) (end 128.805 97.885) (width 1) (layer "F.Cu") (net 1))
 (segment (start 158.2 92.265) (end 167.725 82.74) (width 1) (layer "F.Cu") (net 1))
 (segment (start 134.705 94.17) (end 134.705 99.955) (width 1) (layer "F.Cu") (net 1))
 (segment (start 158.835 30.67) (end 157.47 29.305) (width 1) (layer "F.Cu") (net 1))
 (segment (start 134.705 99.955) (end 134.75 100) (width 1) (layer "F.Cu") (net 1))
 (segment (start 167.725 82.74) (end 170.9 82.74) (width 1) (layer "F.Cu") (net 1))
 (segment (start 168.715 30.67) (end 158.835 30.67) (width 1) (layer "F.Cu") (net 1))
 (segment (start 145.725 29.305) (end 138.925 29.305) (width 1) (layer "F.Cu") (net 1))
 (segment (start 157.47 29.305) (end 145.725 29.305) (width 1) (layer "F.Cu") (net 1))
 (via (at 153.12 66.865) (size 0.8) (drill 0.4) (layers "F.Cu" "B.Cu") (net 1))
 (via (at 136.61 92.265) (size 0.8) (drill 0.4) (layers "F.Cu" "B.Cu") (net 1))
 (segment (start 153.12 75.755) (end 153.12 66.865) (width 1) (layer "B.Cu") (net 1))
 (segment (start 136.61 92.265) (end 153.12 75.755) (width 1) (layer "B.Cu") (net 1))
 (segment (start 170.265 101.51) (end 170.265 98.26) (width 1) (layer "F.Cu") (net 7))
 (segment (start 155.435 82.2) (end 162.235 82.2) (width 1) (layer "F.Cu") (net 7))
 (segment (start 156.93 83.06) (end 156.07 82.2) (width 1) (layer "F.Cu") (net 7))
 (segment (start 169.985 97.98) (end 170.265 98.26) (width 1) (layer "F.Cu") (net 7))
 (segment (start 166.36 97.885) (end 162.87 97.885) (width 1) (layer "F.Cu") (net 7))
 (segment (start 166.455 97.98) (end 169.985 97.98) (width 1) (layer "F.Cu") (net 7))
 (segment (start 162.61 98.26) (end 162.235 97.885) (width 0.25) (layer "F.Cu") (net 7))
 (segment (start 155.435 97.885) (end 162.235 97.885) (width 1) (layer "F.Cu") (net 7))
 (segment (start 166.455 97.98) (end 166.36 97.885) (width 1) (layer "F.Cu") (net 7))
 (segment (start 156.93 86.55) (end 156.93 83.06) (width 1) (layer "F.Cu") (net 7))
 (via (at 166.455 97.98) (size 0.8) (drill 0.4) (layers "F.Cu" "B.Cu") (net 7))
 (via (at 156.93 86.55) (size 0.8) (drill 0.4) (layers "F.Cu" "B.Cu") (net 7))
 (segment (start 158.835 89.725) (end 163.28 89.725) (width 1) (layer "B.Cu") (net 7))
 (segment (start 167.725 85.28) (end 163.28 89.725) (width 1) (layer "B.Cu") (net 7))
 (segment (start 166.455 97.98) (end 166.455 92.9) (width 1) (layer "B.Cu") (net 7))
 (segment (start 170.9 85.28) (end 167.725 85.28) (width 1) (layer "B.Cu") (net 7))
 (segment (start 156.93 86.55) (end 156.93 87.82) (width 1) (layer "B.Cu") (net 7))
 (segment (start 156.93 87.82) (end 158.835 89.725) (width 1) (layer "B.Cu") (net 7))
 (segment (start 166.455 92.9) (end 163.28 89.725) (width 1) (layer "B.Cu") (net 7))
 (segment (start 40.725 100.52) (end 42.09 101.885) (width 1) (layer "F.Cu") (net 8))
 (segment (start 73.11 61.785) (end 53.425 61.785) (width 1) (layer "F.Cu") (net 8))
 (segment (start 53.425 61.785) (end 40.725 74.485) (width 1) (layer "F.Cu") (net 8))
 (segment (start 80.505 101.885) (end 87.305 101.885) (width 1) (layer "F.Cu") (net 8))
 (segment (start 122.005 101.885) (end 128.805 101.885) (width 1) (layer "F.Cu") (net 8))
 (segment (start 42.09 101.885) (end 46.85 101.885) (width 1) (layer "F.Cu") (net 8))
 (segment (start 57.87 101.79) (end 53.745 101.79) (width 1) (layer "F.Cu") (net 8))
 (segment (start 105.085 101.885) (end 121.78 101.885) (width 1) (layer "F.Cu") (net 8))
 (segment (start 153.625 104.33) (end 156.07 101.885) (width 1) (layer "F.Cu") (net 8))
 (segment (start 142.6425 80.2) (end 126.45 80.2) (width 1) (layer "F.Cu") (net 8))
 (segment (start 46.85 101.885) (end 53.65 101.885) (width 1) (layer "F.Cu") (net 8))
 (segment (start 53.745 101.79) (end 53.65 101.885) (width 0.25) (layer "F.Cu") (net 8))
 (segment (start 80.505 101.885) (end 75.745 101.885) (width 1) (layer "F.Cu") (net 8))
 (segment (start 75.745 101.885) (end 75.65 101.79) (width 1) (layer "F.Cu") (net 8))
 (segment (start 40.725 74.485) (end 40.725 100.52) (width 1) (layer "F.Cu") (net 8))
 (segment (start 128.805 101.885) (end 131.25 104.33) (width 1) (layer "F.Cu") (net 8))
 (segment (start 155.435 101.885) (end 162.235 101.885) (width 1) (layer "F.Cu") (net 8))
 (segment (start 152.8025 70.04) (end 142.6425 80.2) (width 1) (layer "F.Cu") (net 8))
 (segment (start 170.9 70.04) (end 152.8025 70.04) (width 1) (layer "F.Cu") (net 8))
 (segment (start 82.635 71.31) (end 73.11 61.785) (width 1) (layer "F.Cu") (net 8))
 (segment (start 117.56 71.31) (end 82.635 71.31) (width 1) (layer "F.Cu") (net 8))
 (segment (start 131.25 104.33) (end 153.625 104.33) (width 1) (layer "F.Cu") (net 8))
 (segment (start 87.305 101.885) (end 98.285 101.885) (width 1) (layer "F.Cu") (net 8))
 (segment (start 98.285 101.885) (end 105.085 101.885) (width 1) (layer "F.Cu") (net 8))
 (segment (start 126.45 80.2) (end 117.56 71.31) (width 1) (layer "F.Cu") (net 8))
 (via (at 57.87 101.79) (size 0.8) (drill 0.4) (layers "F.Cu" "B.Cu") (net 8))
 (via (at 75.65 101.79) (size 0.8) (drill 0.4) (layers "F.Cu" "B.Cu") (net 8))
 (segment (start 75.65 101.79) (end 57.87 101.79) (width 1) (layer "B.Cu") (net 8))
 (segment (start 116.925 73.215) (end 88.6675 73.215) (width 1) (layer "F.Cu") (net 2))
 (segment (start 87.305 74.5775) (end 87.305 82.645) (width 1) (layer "F.Cu") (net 2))
 (segment (start 58.505 77.025) (end 57.33 78.2) (width 1) (layer "F.Cu") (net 2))
 (segment (start 57.33 78.2) (end 53.65 78.2) (width 1) (layer "F.Cu") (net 2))
 (segment (start 59.68 70.77) (end 58.505 71.945) (width 1) (layer "F.Cu") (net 2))
 (segment (start 163.28 72.58) (end 163.055 72.805) (width 0.25) (layer "F.Cu") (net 2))
 (segment (start 153.12 72.58) (end 143.595 82.105) (width 1) (layer "F.Cu") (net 2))
 (segment (start 80.505 82.645) (end 87.305 82.645) (width 1) (layer "F.Cu") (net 2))
 (segment (start 88.6675 73.215) (end 87.305 74.5775) (width 1) (layer "F.Cu") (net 2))
 (segment (start 63.36 70.77) (end 70.16 70.77) (width 1) (layer "F.Cu") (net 2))
 (segment (start 163.28 72.58) (end 170.9 72.58) (width 1) (layer "F.Cu") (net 2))
 (segment (start 163.055 72.805) (end 155.435 72.805) (width 0.25) (layer "F.Cu") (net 2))
 (segment (start 58.505 71.945) (end 58.505 77.025) (width 1) (layer "F.Cu") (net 2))
 (segment (start 76.38 70.77) (end 80.505 74.895) (width 1) (layer "F.Cu") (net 2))
 (segment (start 155.66 72.58) (end 156.07 72.99) (width 1) (layer "F.Cu") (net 2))
 (segment (start 163.28 72.58) (end 155.66 72.58) (width 1) (layer "F.Cu") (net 2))
 (segment (start 80.505 74.895) (end 80.505 82.645) (width 1) (layer "F.Cu") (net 2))
 (segment (start 63.36 70.77) (end 59.68 70.77) (width 1) (layer "F.Cu") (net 2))
 (segment (start 145.725 33.305) (end 138.925 33.305) (width 1) (layer "F.Cu") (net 2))
 (segment (start 151.945 33.305) (end 145.725 33.305) (width 1) (layer "F.Cu") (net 2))
 (segment (start 155.66 72.58) (end 153.12 72.58) (width 1) (layer "F.Cu") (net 2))
 (segment (start 46.85 78.2) (end 53.65 78.2) (width 1) (layer "F.Cu") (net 2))
 (segment (start 125.815 82.105) (end 116.925 73.215) (width 1) (layer "F.Cu") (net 2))
 (segment (start 156.07 72.99) (end 156.07 78.2) (width 1) (layer "F.Cu") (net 2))
 (segment (start 155.435 78.2) (end 162.235 78.2) (width 1) (layer "F.Cu") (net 2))
 (segment (start 163.28 44.64) (end 151.945 33.305) (width 1) (layer "F.Cu") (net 2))
 (segment (start 143.595 82.105) (end 125.815 82.105) (width 1) (layer "F.Cu") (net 2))
 (segment (start 70.16 70.77) (end 76.38 70.77) (width 1) (layer "F.Cu") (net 2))
 (via (at 163.28 72.58) (size 0.8) (drill 0.4) (layers "F.Cu" "B.Cu") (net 2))
 (via (at 163.28 44.64) (size 0.8) (drill 0.4) (layers "F.Cu" "B.Cu") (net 2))
 (segment (start 163.28 44.64) (end 163.28 72.58) (width 1) (layer "B.Cu") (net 2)))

